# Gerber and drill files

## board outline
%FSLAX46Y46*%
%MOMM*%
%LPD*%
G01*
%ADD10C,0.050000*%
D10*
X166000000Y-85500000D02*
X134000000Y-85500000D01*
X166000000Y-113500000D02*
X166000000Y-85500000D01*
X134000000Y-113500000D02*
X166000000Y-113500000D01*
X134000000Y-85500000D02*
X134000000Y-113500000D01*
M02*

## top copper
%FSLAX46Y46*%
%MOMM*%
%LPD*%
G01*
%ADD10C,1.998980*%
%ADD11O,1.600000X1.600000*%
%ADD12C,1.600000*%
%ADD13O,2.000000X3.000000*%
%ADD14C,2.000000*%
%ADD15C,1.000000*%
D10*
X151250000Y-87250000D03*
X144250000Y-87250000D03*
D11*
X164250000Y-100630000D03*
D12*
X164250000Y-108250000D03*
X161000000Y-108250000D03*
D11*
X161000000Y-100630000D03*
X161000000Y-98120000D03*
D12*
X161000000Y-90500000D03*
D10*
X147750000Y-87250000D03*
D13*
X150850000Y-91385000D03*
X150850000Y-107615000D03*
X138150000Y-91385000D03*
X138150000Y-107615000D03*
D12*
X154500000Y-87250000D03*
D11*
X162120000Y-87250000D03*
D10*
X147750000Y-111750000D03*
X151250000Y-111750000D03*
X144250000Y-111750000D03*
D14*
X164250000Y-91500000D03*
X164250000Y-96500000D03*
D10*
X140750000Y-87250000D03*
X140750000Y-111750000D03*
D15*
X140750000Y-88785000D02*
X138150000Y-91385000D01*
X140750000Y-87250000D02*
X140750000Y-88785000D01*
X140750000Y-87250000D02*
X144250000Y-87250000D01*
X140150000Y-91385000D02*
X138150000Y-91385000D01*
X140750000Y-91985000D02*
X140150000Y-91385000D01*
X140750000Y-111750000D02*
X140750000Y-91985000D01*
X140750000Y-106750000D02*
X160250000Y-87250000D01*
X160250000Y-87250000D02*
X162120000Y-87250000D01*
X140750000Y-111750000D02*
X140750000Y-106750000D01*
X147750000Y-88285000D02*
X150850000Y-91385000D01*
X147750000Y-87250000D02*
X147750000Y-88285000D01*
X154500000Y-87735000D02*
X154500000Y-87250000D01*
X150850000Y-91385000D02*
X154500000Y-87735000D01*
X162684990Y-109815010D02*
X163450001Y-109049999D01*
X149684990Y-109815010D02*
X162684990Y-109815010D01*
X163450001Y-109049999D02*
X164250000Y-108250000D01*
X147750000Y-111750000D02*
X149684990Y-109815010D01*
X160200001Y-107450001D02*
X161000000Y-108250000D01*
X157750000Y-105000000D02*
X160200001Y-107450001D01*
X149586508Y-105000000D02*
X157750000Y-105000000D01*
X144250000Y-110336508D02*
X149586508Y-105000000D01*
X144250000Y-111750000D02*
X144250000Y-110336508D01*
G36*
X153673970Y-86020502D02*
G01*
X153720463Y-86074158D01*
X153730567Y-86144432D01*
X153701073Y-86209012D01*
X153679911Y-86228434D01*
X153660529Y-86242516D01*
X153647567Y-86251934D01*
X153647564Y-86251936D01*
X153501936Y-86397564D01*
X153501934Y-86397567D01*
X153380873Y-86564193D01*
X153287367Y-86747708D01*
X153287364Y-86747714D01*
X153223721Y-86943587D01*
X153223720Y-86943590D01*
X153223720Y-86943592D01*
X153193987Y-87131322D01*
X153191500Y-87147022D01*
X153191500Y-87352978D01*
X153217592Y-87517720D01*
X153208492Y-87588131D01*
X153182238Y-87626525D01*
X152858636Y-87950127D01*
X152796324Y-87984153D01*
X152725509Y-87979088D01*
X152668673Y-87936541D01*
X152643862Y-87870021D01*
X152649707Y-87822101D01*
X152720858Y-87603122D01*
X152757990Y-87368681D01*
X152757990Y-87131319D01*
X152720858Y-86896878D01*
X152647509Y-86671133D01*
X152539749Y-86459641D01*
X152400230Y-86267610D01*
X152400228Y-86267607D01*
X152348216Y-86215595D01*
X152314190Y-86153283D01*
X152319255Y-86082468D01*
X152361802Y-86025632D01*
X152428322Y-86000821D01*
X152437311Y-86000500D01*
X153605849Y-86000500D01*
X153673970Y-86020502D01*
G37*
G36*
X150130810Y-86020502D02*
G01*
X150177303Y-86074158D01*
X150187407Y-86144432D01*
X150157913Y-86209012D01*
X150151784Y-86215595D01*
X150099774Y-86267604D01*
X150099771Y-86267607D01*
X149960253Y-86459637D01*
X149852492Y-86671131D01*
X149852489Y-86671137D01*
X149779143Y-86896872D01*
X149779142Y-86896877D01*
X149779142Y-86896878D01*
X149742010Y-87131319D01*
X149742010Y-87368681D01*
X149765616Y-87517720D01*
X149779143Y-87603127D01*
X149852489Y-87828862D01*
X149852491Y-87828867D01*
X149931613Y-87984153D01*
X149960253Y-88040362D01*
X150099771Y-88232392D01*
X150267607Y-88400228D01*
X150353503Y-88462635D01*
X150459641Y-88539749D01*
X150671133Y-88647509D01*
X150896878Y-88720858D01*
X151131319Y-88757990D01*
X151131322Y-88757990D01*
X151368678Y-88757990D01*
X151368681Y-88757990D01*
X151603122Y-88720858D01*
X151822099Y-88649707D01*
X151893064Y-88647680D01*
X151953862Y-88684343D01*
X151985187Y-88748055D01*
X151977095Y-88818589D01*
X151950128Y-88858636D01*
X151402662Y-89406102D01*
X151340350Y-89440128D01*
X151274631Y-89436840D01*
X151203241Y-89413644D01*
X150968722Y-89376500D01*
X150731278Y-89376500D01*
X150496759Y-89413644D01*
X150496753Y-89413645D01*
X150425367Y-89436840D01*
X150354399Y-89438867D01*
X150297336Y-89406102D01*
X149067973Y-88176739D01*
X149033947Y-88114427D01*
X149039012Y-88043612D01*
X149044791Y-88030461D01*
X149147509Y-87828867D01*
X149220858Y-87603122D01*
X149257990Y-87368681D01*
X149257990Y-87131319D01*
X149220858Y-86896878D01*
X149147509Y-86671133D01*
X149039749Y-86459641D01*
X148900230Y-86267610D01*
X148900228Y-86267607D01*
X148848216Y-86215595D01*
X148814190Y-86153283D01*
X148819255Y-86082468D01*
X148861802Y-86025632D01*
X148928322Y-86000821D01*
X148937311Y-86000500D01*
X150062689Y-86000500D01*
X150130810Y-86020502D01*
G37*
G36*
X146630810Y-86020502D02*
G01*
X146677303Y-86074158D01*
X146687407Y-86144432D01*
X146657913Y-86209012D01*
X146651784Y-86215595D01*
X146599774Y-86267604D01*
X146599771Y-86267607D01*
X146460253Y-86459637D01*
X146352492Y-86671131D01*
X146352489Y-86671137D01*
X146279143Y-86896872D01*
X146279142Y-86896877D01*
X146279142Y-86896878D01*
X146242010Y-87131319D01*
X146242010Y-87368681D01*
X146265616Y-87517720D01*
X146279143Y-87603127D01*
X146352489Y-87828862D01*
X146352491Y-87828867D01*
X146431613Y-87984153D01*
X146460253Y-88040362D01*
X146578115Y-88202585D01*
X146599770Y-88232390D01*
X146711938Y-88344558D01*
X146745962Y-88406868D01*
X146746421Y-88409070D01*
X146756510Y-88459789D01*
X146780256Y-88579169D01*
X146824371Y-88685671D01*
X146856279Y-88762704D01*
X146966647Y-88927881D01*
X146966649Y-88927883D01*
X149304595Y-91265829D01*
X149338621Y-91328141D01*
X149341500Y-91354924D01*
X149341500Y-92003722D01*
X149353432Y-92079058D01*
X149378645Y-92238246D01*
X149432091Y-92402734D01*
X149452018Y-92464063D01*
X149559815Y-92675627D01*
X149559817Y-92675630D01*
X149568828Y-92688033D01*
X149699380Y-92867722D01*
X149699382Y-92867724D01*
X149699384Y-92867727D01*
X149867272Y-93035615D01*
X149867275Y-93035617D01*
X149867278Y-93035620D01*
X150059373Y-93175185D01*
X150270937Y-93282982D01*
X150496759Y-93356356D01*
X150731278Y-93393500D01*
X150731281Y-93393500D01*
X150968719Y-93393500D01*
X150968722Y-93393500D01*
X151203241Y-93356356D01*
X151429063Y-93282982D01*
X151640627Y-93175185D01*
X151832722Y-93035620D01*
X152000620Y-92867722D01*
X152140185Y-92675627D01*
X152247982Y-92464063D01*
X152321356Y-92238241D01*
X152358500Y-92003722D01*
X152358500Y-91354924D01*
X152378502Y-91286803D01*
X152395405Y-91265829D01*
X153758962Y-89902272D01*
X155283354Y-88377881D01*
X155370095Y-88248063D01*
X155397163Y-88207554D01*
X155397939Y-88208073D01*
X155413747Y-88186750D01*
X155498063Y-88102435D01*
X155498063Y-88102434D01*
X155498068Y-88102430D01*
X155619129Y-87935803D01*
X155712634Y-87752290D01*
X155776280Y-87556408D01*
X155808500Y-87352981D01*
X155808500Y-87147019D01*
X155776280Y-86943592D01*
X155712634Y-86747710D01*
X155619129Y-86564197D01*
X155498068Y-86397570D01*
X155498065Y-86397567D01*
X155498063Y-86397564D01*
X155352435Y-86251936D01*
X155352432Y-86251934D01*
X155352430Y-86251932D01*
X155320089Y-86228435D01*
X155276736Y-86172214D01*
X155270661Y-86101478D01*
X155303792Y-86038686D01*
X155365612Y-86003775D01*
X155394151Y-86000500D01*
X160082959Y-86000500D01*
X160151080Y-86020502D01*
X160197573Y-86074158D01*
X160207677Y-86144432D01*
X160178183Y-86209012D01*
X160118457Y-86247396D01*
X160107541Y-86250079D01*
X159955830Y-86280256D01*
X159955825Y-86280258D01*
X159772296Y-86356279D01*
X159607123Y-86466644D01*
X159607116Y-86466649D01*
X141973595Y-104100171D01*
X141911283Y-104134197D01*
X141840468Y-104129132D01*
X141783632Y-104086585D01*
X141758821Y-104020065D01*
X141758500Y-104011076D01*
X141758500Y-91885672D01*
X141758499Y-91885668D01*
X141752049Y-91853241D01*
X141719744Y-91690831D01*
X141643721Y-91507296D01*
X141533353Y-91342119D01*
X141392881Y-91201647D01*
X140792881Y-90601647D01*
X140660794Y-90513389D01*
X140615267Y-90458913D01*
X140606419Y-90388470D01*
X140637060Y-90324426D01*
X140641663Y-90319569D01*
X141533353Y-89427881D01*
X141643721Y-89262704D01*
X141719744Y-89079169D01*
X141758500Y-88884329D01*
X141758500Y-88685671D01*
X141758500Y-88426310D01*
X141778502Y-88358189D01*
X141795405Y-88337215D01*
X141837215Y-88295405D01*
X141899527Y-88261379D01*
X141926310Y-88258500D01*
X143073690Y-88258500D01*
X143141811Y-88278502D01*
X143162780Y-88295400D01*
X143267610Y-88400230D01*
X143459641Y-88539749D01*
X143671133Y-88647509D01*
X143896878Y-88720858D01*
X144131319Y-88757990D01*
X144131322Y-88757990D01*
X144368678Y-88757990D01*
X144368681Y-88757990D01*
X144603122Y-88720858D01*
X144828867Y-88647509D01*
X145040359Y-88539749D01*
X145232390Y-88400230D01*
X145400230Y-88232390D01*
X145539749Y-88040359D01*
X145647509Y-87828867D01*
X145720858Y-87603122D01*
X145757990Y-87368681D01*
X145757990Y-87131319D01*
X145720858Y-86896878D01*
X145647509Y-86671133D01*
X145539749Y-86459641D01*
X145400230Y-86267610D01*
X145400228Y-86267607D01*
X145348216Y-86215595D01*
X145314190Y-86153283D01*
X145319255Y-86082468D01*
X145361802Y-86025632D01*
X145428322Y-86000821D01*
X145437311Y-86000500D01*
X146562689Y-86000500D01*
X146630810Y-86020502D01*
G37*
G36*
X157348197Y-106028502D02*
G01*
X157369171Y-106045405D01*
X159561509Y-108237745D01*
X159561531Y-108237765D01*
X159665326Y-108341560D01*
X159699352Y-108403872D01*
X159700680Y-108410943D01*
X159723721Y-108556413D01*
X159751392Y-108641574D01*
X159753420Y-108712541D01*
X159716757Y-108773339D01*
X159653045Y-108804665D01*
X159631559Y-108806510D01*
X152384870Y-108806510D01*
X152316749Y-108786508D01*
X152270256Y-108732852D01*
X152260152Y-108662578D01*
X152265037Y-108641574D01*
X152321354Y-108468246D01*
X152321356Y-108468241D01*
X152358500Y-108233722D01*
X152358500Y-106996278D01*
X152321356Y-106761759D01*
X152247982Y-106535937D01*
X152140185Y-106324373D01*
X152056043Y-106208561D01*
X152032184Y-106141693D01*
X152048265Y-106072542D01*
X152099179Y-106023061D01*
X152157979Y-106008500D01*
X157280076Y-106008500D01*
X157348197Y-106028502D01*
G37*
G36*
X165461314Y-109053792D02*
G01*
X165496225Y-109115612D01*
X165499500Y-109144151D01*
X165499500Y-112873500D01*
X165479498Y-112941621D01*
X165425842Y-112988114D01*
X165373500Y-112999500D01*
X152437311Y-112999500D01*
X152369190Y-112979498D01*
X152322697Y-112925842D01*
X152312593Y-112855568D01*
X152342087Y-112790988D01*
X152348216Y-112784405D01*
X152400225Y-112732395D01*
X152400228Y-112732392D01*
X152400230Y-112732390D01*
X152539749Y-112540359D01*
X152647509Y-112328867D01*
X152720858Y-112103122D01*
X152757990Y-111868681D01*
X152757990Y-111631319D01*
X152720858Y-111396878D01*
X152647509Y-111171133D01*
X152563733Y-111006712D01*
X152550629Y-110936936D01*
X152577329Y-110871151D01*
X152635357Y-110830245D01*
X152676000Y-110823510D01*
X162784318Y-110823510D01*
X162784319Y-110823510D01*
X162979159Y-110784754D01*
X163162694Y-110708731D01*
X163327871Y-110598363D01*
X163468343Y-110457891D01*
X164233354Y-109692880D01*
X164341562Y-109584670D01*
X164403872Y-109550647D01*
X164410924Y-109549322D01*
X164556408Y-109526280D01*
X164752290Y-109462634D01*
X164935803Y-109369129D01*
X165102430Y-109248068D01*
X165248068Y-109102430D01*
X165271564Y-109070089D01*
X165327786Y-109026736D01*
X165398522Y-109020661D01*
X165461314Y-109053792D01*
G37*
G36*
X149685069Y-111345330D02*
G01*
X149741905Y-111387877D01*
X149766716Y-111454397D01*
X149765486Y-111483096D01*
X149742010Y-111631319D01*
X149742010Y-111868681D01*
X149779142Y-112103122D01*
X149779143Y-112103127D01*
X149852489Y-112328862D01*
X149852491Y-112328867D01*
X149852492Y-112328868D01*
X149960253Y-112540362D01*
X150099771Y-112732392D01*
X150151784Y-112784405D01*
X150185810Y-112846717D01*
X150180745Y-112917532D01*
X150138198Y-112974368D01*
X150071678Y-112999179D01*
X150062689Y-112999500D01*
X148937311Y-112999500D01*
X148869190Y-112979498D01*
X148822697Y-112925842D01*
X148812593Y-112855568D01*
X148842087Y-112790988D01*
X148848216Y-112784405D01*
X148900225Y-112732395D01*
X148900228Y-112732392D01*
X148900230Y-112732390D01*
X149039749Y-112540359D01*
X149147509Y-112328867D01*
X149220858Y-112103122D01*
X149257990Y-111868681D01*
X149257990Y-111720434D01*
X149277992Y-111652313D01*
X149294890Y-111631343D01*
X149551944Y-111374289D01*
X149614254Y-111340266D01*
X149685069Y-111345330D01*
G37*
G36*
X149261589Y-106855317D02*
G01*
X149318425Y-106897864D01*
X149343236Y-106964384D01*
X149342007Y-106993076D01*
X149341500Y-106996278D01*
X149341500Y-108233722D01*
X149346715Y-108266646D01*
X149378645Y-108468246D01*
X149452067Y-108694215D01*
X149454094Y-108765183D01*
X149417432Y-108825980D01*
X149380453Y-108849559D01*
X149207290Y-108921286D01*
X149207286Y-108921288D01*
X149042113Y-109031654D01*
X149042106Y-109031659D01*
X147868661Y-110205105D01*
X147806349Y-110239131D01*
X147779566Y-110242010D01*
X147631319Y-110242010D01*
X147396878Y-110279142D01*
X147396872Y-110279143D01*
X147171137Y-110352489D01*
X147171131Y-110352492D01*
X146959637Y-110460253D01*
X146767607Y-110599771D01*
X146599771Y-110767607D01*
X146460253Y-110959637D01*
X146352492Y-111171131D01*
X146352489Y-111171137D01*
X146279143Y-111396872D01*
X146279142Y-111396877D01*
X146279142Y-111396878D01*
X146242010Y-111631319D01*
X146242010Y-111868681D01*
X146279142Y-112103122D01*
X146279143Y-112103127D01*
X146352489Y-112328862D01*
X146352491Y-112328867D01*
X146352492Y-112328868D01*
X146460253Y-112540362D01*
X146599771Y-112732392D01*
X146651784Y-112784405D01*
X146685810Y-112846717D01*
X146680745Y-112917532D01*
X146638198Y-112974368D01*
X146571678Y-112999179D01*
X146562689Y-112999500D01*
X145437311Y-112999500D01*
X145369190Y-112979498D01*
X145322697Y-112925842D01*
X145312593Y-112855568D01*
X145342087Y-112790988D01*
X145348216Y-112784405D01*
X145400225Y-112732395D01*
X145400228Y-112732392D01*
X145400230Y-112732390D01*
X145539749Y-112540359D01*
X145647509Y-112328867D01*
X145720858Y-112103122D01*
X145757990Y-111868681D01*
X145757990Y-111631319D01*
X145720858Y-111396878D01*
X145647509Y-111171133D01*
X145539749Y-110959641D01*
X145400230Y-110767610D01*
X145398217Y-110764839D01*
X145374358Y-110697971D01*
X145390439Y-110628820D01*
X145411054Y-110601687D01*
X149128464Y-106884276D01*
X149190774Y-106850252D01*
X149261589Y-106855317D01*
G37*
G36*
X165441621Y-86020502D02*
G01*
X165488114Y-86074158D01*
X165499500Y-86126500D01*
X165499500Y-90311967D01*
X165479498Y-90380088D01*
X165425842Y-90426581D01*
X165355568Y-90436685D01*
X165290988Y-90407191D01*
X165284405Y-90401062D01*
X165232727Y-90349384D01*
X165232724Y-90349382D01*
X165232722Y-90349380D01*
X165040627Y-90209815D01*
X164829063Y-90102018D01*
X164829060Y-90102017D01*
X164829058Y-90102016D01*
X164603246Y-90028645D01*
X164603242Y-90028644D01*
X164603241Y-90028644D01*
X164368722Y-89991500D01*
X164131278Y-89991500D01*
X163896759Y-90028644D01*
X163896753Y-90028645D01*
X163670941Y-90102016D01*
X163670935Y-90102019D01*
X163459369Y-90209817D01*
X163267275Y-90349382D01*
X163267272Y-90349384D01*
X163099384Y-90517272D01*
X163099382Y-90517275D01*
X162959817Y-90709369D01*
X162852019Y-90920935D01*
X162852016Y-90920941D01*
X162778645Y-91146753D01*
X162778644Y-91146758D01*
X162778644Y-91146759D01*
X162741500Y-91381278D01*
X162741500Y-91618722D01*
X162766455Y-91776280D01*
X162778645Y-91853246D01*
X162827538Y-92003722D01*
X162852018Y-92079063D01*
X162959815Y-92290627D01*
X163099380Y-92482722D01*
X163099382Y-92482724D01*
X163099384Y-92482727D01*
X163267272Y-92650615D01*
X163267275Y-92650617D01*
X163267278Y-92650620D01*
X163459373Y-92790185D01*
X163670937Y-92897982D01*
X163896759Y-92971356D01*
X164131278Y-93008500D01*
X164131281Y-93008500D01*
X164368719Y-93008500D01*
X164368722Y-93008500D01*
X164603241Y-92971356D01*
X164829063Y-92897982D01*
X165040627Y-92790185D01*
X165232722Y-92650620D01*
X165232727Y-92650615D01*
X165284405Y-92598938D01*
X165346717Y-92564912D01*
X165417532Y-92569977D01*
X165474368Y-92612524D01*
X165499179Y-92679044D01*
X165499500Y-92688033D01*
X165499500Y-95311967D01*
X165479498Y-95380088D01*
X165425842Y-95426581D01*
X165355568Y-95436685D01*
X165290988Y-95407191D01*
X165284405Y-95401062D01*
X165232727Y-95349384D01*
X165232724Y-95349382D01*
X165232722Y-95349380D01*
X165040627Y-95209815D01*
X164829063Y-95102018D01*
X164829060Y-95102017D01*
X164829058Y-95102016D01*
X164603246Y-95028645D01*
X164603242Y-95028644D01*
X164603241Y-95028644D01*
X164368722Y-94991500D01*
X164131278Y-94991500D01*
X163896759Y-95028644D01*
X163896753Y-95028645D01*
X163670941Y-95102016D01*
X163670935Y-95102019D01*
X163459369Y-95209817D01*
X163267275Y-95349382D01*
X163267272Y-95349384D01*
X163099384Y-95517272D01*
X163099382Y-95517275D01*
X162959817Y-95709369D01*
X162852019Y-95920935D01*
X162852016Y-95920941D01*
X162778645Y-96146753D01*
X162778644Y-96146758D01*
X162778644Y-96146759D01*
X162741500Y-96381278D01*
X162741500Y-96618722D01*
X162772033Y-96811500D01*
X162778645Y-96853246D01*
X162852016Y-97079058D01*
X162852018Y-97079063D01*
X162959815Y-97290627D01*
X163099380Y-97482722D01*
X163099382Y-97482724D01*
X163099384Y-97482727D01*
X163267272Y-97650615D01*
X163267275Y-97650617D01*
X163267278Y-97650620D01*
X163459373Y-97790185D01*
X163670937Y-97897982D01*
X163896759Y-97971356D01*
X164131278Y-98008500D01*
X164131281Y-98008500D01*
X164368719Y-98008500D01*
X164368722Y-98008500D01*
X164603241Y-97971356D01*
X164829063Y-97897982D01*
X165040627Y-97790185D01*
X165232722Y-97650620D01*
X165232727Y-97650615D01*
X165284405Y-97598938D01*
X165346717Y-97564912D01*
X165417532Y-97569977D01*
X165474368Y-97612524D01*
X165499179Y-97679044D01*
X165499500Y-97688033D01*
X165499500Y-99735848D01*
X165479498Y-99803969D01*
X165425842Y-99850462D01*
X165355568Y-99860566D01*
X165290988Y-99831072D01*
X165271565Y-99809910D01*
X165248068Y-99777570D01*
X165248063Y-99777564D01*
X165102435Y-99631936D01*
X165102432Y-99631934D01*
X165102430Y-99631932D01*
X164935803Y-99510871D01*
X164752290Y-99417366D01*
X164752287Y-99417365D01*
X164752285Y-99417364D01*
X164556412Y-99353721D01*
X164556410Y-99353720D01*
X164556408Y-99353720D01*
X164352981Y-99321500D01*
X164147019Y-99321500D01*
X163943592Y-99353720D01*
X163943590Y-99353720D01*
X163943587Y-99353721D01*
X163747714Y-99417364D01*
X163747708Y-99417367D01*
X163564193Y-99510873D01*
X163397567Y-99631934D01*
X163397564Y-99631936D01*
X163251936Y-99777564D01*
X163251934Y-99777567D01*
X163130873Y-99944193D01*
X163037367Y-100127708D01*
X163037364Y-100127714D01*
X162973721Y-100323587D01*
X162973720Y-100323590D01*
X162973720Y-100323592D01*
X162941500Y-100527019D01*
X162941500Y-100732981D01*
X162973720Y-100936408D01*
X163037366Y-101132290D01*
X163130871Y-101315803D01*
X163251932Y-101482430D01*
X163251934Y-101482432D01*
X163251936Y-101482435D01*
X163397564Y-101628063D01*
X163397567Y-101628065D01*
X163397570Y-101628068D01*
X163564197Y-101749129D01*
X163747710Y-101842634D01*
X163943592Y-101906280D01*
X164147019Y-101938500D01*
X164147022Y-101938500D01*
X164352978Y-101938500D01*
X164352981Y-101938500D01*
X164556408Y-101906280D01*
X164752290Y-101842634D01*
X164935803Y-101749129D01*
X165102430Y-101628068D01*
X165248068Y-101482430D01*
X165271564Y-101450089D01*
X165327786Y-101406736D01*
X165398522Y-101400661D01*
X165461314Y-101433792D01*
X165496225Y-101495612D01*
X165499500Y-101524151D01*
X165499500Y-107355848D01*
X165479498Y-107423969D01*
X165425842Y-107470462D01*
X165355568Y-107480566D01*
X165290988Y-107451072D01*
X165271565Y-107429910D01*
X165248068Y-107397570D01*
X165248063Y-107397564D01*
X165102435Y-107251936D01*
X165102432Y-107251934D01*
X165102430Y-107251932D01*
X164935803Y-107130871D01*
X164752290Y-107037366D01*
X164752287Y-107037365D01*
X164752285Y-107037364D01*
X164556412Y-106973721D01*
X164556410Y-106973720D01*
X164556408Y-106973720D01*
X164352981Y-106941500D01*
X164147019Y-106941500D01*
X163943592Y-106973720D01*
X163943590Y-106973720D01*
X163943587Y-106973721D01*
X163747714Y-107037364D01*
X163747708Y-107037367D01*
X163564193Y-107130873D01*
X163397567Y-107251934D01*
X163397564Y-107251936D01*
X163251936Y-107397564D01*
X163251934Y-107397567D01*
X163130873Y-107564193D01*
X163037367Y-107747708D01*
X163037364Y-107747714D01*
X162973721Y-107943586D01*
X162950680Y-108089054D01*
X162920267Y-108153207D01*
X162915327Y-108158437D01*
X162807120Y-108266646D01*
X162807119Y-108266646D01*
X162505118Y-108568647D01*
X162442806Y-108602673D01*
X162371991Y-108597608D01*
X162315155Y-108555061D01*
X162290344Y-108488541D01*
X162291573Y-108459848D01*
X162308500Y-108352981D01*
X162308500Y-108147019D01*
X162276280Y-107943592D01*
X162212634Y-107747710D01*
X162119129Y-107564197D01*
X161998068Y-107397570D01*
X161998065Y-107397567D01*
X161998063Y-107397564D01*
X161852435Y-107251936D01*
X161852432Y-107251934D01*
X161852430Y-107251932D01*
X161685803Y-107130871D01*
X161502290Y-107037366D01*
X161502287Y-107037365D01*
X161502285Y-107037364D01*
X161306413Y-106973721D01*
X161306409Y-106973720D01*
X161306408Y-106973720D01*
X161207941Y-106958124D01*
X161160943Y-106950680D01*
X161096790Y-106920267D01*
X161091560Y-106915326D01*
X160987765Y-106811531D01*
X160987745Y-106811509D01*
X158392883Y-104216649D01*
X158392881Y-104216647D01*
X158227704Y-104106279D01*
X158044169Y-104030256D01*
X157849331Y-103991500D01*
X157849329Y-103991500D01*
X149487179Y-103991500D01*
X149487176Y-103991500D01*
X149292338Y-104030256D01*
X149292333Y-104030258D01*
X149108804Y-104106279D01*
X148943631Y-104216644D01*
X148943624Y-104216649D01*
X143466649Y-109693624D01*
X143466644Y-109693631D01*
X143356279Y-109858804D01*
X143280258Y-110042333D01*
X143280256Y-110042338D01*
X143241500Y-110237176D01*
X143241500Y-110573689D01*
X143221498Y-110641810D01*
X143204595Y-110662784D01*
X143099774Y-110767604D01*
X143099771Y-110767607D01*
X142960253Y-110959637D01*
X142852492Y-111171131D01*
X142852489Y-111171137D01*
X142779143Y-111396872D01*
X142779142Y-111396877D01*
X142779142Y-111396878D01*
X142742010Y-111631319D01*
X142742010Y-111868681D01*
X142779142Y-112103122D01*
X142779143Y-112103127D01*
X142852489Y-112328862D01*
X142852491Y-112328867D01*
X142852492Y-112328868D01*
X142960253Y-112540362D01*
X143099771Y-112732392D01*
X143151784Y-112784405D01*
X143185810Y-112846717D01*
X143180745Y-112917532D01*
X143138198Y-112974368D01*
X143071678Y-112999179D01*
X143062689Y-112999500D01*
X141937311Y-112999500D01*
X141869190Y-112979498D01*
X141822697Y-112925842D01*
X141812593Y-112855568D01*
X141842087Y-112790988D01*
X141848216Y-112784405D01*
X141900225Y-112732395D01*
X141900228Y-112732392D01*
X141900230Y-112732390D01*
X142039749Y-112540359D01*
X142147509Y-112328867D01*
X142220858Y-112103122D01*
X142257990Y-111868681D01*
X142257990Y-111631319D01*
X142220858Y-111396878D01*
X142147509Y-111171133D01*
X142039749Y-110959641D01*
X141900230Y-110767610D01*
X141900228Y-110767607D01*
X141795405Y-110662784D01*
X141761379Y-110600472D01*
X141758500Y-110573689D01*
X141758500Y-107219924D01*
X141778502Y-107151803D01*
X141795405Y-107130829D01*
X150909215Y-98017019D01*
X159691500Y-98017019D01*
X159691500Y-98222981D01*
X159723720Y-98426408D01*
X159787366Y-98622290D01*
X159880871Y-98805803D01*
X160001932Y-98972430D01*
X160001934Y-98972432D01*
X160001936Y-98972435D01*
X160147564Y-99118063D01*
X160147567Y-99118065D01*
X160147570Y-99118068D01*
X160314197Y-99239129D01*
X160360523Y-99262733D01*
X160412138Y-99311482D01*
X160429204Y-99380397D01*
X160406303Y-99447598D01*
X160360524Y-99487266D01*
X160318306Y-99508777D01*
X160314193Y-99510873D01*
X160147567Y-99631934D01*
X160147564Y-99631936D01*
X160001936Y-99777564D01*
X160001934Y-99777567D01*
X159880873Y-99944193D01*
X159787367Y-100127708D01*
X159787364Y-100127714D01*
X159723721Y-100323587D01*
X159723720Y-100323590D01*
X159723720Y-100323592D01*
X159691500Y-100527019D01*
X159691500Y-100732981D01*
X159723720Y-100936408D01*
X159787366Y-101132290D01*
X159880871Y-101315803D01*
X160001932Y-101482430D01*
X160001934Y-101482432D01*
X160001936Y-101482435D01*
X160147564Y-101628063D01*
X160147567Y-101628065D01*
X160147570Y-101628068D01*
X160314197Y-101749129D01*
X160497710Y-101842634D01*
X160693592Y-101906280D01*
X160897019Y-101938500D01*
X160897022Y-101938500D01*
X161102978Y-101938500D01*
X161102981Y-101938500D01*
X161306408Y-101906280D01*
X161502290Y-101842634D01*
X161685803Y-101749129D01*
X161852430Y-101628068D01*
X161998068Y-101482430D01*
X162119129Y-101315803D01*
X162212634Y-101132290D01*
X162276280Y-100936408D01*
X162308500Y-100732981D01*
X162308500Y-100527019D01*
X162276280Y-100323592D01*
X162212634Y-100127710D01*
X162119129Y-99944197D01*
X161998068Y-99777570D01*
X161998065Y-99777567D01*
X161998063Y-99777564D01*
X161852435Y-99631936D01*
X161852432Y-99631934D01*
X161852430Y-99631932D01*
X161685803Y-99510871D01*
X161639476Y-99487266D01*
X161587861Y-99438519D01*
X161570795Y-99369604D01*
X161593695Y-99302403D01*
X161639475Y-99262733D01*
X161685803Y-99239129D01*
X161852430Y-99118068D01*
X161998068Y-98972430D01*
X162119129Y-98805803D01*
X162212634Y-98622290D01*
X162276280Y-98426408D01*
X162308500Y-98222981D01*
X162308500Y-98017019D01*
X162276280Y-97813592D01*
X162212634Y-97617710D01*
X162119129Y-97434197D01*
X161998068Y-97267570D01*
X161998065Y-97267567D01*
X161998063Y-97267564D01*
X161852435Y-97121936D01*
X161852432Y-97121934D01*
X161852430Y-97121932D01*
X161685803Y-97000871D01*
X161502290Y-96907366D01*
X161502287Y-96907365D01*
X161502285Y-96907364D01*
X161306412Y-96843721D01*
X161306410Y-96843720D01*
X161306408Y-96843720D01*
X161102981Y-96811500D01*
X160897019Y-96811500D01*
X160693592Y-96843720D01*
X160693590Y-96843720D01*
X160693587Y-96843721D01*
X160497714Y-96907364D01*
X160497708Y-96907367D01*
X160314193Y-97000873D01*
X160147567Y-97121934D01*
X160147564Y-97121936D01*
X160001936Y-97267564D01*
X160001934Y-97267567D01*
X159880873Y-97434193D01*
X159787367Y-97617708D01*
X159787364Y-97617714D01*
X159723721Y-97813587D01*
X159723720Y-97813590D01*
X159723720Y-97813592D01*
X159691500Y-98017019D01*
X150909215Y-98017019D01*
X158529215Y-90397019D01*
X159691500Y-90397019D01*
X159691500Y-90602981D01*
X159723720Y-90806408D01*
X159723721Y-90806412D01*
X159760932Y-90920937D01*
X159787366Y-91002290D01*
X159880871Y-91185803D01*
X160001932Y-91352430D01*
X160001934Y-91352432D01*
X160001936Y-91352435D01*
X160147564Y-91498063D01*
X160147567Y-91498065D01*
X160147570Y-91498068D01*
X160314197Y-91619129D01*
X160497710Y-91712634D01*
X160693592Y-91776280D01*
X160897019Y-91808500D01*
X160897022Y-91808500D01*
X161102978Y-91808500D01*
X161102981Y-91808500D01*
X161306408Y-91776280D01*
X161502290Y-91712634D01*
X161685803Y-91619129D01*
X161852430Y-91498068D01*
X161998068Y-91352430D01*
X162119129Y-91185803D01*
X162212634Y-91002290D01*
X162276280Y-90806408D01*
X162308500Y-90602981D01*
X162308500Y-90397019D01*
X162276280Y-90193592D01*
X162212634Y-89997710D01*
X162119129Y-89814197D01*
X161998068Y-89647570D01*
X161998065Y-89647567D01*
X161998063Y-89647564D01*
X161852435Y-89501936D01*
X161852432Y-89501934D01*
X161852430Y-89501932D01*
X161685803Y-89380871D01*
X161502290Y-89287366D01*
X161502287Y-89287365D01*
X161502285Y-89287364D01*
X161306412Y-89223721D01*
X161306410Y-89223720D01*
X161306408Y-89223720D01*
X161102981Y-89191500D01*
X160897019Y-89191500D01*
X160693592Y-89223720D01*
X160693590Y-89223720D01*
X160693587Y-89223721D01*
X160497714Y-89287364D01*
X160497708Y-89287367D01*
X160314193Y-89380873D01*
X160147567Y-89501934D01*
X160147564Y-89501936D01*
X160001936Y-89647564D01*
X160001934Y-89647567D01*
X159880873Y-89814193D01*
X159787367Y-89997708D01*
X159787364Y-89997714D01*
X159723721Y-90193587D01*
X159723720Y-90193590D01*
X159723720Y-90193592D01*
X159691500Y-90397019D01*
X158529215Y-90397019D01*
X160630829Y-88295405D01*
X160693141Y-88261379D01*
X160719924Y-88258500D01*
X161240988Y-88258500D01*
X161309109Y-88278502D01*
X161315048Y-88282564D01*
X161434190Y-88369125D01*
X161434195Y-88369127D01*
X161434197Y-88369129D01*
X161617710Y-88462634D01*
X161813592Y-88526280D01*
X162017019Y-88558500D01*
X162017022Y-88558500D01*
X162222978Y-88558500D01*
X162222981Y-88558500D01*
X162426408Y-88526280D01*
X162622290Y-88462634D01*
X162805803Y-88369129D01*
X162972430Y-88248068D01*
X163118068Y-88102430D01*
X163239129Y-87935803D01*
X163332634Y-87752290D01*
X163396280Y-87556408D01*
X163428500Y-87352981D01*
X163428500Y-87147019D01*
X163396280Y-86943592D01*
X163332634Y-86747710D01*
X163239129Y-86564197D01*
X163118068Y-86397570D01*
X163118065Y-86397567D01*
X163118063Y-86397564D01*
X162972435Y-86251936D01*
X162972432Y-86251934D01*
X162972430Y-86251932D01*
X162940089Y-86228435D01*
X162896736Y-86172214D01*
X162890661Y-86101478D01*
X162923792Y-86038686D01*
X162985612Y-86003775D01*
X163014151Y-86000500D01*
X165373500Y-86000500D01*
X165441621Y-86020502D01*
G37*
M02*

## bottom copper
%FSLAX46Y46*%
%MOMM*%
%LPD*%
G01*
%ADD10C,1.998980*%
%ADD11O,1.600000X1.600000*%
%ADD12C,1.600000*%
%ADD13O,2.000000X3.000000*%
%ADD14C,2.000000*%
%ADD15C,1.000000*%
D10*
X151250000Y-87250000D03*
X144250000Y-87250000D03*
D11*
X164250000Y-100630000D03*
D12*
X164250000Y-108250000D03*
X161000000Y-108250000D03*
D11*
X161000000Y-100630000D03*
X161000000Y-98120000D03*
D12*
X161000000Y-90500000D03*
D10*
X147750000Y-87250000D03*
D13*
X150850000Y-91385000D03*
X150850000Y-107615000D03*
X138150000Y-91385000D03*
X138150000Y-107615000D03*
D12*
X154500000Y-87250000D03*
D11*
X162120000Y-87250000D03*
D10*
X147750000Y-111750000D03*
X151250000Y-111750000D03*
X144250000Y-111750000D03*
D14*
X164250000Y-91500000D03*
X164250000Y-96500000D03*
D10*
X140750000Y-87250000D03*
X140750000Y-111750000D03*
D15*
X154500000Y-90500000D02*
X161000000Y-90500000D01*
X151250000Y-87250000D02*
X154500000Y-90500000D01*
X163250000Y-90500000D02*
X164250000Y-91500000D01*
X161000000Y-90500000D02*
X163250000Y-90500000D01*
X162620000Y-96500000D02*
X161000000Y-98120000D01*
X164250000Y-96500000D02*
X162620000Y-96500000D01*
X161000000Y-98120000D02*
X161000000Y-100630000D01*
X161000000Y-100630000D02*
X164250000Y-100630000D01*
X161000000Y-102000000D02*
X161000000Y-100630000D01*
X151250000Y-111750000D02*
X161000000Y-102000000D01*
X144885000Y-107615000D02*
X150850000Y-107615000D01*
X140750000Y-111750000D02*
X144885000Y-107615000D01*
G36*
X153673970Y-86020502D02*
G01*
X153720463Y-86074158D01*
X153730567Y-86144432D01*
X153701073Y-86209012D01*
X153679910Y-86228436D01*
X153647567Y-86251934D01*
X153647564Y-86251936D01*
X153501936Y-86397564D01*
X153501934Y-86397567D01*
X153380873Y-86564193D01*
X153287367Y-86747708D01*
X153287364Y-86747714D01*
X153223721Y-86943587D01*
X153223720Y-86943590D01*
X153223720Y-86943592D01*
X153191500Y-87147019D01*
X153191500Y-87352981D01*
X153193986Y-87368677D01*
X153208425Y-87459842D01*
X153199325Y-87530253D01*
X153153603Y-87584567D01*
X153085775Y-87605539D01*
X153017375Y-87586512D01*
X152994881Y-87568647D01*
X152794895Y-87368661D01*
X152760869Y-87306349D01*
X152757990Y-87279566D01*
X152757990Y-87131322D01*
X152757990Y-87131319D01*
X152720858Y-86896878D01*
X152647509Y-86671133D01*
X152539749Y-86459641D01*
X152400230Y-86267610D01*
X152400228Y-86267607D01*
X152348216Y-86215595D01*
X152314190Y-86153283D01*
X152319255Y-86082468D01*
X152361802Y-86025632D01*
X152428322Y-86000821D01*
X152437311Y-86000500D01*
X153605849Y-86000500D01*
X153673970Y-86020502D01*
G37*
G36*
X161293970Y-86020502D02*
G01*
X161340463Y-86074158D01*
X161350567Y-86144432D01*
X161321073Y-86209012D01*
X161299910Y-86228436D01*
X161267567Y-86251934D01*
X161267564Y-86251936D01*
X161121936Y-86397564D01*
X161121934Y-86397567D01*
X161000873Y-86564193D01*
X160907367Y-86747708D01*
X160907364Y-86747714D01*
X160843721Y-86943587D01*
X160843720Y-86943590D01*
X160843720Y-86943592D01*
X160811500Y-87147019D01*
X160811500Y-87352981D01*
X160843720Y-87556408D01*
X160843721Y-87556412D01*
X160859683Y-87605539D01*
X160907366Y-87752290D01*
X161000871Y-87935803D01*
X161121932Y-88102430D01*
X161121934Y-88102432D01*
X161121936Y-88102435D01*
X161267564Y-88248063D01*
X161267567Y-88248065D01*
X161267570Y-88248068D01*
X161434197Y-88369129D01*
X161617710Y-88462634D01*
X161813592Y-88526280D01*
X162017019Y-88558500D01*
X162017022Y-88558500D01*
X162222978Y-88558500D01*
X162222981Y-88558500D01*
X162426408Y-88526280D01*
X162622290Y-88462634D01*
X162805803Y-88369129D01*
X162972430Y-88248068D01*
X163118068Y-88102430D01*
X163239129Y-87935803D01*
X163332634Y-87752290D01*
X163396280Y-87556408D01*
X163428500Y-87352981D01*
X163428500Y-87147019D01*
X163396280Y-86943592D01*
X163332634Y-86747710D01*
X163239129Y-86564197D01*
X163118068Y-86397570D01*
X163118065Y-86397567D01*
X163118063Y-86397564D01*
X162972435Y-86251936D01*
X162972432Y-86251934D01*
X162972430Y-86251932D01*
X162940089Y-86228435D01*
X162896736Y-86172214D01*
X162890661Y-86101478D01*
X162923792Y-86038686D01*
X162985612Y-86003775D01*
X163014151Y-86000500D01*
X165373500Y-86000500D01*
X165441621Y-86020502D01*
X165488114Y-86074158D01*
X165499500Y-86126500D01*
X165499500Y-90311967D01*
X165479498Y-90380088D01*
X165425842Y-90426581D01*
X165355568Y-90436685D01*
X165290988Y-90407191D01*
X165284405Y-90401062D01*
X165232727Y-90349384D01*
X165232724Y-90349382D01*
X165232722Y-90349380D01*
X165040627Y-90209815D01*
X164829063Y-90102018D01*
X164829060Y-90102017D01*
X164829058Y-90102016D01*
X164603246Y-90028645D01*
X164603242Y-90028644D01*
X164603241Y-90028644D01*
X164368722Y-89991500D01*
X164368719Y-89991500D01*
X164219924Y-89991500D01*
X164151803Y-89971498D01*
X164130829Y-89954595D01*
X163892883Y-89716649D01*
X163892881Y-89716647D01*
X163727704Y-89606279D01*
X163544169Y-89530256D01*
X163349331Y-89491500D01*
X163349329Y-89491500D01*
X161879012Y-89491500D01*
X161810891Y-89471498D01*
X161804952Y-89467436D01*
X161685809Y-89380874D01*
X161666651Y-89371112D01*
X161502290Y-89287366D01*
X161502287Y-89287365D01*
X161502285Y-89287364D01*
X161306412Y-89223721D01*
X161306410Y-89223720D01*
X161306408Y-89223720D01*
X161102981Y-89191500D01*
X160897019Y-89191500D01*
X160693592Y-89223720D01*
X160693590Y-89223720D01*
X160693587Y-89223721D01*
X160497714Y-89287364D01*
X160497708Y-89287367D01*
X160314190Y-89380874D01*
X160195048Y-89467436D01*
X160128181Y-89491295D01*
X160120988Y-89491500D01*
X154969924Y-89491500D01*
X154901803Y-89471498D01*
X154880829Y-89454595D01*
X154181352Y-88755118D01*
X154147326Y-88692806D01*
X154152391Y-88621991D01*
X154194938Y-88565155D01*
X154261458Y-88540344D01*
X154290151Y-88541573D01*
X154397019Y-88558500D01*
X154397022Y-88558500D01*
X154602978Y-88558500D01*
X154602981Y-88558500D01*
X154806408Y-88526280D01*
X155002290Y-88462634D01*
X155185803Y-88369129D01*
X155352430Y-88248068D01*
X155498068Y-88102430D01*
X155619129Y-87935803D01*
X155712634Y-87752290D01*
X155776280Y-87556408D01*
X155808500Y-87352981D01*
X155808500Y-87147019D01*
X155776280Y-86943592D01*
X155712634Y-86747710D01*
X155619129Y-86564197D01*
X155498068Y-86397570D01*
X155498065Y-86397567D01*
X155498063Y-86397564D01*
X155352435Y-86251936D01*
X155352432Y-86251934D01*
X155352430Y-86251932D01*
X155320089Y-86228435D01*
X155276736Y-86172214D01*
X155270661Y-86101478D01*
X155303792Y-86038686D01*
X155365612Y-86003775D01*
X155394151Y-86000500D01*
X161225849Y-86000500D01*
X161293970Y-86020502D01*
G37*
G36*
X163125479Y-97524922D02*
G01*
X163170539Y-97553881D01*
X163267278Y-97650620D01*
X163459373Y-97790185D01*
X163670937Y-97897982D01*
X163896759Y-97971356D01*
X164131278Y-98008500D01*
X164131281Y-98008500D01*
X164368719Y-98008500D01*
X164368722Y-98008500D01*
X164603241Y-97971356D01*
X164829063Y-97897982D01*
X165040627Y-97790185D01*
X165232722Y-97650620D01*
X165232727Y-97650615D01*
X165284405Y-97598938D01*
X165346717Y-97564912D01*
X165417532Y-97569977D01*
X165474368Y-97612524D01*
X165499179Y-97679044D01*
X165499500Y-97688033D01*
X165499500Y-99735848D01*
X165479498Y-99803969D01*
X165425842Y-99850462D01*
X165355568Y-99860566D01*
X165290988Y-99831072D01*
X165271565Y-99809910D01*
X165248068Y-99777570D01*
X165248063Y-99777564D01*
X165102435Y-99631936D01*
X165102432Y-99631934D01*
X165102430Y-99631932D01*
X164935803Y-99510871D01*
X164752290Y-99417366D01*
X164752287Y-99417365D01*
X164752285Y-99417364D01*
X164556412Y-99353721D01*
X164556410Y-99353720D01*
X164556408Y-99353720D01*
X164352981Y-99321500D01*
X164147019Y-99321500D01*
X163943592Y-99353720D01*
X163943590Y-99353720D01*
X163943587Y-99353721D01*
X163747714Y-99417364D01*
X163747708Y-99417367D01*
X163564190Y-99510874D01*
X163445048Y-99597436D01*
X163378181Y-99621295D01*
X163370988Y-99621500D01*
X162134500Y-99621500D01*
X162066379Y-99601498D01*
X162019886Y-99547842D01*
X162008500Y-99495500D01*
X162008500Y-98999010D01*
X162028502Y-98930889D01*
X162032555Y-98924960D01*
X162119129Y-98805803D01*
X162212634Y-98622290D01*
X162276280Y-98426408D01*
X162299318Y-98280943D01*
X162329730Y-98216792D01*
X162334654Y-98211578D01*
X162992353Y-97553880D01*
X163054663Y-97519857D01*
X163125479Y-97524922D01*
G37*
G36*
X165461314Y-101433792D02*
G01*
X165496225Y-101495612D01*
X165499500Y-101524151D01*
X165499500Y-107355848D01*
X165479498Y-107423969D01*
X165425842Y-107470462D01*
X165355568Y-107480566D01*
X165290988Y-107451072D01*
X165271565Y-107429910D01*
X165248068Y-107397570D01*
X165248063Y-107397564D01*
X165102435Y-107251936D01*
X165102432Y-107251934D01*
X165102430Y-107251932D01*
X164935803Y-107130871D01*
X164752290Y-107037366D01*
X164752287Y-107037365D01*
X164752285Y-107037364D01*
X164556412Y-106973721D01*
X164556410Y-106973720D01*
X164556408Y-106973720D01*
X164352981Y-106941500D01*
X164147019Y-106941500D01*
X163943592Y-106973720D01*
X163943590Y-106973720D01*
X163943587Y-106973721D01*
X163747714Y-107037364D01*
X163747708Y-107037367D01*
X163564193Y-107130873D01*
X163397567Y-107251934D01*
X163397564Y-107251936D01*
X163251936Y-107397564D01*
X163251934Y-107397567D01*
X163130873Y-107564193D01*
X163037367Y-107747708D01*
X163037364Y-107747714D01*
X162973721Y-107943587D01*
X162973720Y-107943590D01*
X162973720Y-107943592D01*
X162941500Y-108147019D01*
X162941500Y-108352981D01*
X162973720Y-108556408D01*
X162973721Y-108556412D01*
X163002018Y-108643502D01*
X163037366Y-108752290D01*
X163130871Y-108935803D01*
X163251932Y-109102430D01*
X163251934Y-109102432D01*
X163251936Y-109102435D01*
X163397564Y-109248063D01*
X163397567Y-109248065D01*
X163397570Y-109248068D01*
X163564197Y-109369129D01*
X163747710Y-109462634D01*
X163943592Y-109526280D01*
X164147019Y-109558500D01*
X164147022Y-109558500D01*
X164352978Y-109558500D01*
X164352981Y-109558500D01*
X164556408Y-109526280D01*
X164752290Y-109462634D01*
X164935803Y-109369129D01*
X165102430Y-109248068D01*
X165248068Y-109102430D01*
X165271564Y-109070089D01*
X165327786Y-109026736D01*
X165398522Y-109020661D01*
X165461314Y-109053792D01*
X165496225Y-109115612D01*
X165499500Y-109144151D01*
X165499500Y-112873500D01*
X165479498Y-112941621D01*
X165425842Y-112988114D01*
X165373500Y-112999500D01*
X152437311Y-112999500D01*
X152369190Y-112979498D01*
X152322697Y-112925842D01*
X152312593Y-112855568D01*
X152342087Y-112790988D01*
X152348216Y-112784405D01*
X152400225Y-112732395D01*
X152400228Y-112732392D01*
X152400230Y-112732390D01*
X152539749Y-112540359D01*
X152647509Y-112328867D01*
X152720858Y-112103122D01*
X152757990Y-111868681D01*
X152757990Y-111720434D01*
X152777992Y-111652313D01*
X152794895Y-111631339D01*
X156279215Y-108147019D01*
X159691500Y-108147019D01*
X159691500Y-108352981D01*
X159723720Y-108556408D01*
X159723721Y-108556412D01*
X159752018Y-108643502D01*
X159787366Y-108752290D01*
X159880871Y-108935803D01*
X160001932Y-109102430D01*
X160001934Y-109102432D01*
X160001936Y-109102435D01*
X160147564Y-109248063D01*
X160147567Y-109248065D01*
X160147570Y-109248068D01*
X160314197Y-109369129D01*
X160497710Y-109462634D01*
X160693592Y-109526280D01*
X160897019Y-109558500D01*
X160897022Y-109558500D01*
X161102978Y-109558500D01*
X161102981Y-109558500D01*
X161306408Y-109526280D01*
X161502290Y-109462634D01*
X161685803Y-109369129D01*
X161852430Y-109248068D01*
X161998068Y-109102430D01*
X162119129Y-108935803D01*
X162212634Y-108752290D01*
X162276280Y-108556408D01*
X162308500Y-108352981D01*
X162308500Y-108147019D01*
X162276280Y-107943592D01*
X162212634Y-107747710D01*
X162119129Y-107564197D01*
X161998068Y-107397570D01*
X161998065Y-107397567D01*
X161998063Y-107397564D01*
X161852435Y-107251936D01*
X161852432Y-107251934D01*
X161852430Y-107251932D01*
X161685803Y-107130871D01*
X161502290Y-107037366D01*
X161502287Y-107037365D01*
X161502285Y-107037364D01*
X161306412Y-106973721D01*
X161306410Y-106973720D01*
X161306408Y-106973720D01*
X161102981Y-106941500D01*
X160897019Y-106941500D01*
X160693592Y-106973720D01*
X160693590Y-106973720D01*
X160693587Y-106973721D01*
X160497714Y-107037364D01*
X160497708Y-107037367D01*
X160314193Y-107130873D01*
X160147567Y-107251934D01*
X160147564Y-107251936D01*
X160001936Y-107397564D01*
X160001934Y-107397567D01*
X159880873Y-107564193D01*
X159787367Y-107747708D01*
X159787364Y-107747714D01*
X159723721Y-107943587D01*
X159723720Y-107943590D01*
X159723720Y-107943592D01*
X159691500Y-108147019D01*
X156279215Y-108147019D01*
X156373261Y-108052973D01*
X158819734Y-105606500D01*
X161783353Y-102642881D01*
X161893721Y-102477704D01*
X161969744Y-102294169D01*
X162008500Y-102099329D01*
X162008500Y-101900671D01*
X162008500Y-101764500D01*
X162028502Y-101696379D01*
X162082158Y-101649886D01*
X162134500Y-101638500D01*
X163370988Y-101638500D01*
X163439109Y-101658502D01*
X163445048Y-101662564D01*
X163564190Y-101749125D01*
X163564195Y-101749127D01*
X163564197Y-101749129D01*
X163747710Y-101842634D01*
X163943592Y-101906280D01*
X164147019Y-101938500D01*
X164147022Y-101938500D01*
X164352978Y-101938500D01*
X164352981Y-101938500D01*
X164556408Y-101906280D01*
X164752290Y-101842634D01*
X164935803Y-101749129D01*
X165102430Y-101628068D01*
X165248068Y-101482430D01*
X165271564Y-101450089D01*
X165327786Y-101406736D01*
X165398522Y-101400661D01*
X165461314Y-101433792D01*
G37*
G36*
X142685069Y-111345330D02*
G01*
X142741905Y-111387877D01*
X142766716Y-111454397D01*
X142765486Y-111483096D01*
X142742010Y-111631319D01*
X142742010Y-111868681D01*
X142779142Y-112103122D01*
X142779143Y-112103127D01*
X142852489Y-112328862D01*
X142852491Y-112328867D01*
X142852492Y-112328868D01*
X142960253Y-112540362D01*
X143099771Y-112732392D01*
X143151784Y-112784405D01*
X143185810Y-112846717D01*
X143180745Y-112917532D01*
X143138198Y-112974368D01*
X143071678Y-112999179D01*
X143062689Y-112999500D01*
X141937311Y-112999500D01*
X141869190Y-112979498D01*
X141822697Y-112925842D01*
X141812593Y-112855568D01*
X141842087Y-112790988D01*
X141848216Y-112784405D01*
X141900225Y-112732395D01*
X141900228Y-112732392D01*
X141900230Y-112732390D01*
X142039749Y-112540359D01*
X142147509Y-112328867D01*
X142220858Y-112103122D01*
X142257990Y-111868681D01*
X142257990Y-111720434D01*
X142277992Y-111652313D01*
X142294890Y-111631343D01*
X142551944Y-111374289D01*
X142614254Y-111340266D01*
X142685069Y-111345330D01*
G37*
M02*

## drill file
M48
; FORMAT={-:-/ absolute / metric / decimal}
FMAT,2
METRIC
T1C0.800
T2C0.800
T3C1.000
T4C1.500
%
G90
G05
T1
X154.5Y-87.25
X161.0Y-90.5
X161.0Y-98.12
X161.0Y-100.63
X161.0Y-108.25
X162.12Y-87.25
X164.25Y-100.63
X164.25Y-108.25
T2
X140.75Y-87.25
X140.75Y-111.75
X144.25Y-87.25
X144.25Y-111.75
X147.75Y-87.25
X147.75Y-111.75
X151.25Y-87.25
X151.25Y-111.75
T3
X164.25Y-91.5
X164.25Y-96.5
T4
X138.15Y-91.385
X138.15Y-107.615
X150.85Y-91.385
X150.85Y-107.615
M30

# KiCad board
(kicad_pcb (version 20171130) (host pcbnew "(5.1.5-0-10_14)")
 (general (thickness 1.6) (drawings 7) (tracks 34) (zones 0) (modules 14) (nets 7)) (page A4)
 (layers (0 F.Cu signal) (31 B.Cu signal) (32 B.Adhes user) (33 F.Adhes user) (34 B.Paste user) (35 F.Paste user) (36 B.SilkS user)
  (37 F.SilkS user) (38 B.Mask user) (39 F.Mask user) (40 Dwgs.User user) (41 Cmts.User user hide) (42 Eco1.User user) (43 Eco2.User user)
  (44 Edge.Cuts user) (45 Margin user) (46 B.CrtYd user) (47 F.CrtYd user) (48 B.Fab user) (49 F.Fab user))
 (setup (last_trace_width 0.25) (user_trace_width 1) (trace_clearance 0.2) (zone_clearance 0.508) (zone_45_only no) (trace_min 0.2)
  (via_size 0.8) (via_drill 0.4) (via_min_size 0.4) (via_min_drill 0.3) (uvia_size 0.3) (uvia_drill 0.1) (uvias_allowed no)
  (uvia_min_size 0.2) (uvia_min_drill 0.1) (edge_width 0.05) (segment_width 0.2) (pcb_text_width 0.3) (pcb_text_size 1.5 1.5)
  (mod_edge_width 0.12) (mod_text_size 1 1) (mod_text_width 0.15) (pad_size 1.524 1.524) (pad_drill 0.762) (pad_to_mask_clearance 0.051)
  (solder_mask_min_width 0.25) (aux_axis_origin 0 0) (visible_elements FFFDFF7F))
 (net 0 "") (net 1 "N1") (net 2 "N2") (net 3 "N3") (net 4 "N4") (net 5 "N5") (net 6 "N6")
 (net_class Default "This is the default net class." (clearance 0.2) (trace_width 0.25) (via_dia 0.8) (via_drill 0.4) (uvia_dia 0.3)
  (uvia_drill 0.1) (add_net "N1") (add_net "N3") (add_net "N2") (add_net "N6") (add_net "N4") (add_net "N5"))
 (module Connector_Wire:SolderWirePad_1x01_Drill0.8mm (layer F.Cu) (at 151.25 87.25 180)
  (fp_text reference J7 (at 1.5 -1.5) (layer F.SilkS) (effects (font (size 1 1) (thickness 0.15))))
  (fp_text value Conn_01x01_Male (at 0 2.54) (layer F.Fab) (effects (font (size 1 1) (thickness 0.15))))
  (pad 1 thru_hole circle (at 0 0 180) (size 1.99898 1.99898) (drill 0.8001) (layers *.Cu *.Mask) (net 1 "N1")))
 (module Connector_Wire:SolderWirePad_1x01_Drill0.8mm (layer F.Cu) (at 144.25 87.25)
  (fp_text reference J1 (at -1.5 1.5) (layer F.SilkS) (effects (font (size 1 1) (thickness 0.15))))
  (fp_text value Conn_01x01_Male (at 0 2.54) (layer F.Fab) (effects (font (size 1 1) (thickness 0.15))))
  (pad 1 thru_hole circle (at 0 0) (size 1.99898 1.99898) (drill 0.8001) (layers *.Cu *.Mask) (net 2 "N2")))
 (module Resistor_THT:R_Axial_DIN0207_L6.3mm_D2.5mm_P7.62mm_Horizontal (layer F.Cu) (at 164.25 108.25 90)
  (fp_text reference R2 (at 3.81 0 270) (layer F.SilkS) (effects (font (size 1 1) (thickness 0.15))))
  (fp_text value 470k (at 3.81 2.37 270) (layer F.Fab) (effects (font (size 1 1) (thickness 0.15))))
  (pad 2 thru_hole oval (at 7.62 0 90) (size 1.6 1.6) (drill 0.8) (layers *.Cu *.Mask) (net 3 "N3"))
  (pad 1 thru_hole circle (at 0 0 90) (size 1.6 1.6) (drill 0.8) (layers *.Cu *.Mask) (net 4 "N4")))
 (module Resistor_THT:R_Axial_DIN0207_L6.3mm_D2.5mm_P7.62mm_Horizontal (layer F.Cu) (at 161 108.25 90)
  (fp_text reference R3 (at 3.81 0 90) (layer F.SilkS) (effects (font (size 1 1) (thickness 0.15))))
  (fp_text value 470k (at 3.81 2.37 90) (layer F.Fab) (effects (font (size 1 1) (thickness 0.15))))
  (pad 1 thru_hole circle (at 0 0 90) (size 1.6 1.6) (drill 0.8) (layers *.Cu *.Mask) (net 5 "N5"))
  (pad 2 thru_hole oval (at 7.62 0 90) (size 1.6 1.6) (drill 0.8) (layers *.Cu *.Mask) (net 3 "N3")))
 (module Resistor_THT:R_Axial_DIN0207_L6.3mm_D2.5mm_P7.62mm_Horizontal (layer F.Cu) (at 161 90.5 270)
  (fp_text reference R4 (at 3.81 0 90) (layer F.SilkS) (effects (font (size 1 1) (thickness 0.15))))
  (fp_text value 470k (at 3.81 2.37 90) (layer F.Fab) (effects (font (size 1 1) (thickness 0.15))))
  (pad 2 thru_hole oval (at 7.62 0 270) (size 1.6 1.6) (drill 0.8) (layers *.Cu *.Mask) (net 3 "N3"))
  (pad 1 thru_hole circle (at 0 0 270) (size 1.6 1.6) (drill 0.8) (layers *.Cu *.Mask) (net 1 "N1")))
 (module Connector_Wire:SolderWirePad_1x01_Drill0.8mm (layer F.Cu) (at 147.75 87.25)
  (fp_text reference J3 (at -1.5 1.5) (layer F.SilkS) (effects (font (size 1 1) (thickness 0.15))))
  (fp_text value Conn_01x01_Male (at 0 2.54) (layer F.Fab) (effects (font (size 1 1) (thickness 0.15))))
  (pad 1 thru_hole circle (at 0 0) (size 1.99898 1.99898) (drill 0.8001) (layers *.Cu *.Mask) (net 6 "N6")))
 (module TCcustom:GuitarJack (layer B.Cu) (at 144.5 99.5 180)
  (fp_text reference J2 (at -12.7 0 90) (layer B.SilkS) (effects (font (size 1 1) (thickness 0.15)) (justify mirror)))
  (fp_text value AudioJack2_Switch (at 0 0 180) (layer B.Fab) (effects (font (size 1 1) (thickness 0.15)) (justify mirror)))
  (pad T thru_hole oval (at -6.35 8.115 180) (size 2 3) (drill 1.5) (layers *.Cu *.Mask) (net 6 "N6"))
  (pad TN thru_hole oval (at -6.35 -8.115 180) (size 2 3) (drill 1.5) (layers *.Cu *.Mask) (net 2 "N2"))
  (pad S thru_hole oval (at 6.35 8.115 180) (size 2 3) (drill 1.5) (layers *.Cu *.Mask) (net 2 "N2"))
  (pad SN thru_hole oval (at 6.35 -8.115 180) (size 2 3) (drill 1.5) (layers *.Cu *.Mask)))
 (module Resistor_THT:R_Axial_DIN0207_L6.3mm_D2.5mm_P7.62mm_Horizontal (layer F.Cu) (at 154.5 87.25)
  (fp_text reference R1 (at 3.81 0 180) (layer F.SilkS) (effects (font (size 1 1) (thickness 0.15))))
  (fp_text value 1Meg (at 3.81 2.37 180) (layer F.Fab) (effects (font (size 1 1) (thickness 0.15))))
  (pad 1 thru_hole circle (at 0 0) (size 1.6 1.6) (drill 0.8) (layers *.Cu *.Mask) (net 6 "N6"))
  (pad 2 thru_hole oval (at 7.62 0) (size 1.6 1.6) (drill 0.8) (layers *.Cu *.Mask) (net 2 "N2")))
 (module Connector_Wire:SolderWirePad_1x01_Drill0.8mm (layer F.Cu) (at 147.75 111.75)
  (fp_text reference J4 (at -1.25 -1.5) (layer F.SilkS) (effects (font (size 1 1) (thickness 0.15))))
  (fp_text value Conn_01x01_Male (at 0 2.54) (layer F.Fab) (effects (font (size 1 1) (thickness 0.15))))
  (pad 1 thru_hole circle (at 0 0) (size 1.99898 1.99898) (drill 0.8001) (layers *.Cu *.Mask) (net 4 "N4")))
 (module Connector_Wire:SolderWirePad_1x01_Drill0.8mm (layer F.Cu) (at 151.25 111.75 180)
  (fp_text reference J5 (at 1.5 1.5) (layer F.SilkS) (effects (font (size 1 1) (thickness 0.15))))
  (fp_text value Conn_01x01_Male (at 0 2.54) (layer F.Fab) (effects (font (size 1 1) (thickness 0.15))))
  (pad 1 thru_hole circle (at 0 0 180) (size 1.99898 1.99898) (drill 0.8001) (layers *.Cu *.Mask) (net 3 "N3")))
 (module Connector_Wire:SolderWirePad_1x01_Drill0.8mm (layer F.Cu) (at 144.25 111.75 180)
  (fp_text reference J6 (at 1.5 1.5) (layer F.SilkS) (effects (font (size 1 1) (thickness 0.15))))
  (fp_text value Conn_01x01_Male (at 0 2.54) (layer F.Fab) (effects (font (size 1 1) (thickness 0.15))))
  (pad 1 thru_hole circle (at 0 0 180) (size 1.99898 1.99898) (drill 0.8001) (layers *.Cu *.Mask) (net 5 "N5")))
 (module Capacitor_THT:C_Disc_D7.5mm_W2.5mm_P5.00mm (layer F.Cu) (at 164.25 91.5 270)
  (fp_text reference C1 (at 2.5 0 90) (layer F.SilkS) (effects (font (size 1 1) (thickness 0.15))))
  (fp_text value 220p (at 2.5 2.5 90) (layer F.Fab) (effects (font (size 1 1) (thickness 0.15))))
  (pad 1 thru_hole circle (at 0 0 270) (size 2 2) (drill 1) (layers *.Cu *.Mask) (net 1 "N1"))
  (pad 2 thru_hole circle (at 5 0 270) (size 2 2) (drill 1) (layers *.Cu *.Mask) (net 3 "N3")))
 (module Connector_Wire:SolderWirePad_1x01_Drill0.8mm (layer F.Cu) (at 140.75 87.25)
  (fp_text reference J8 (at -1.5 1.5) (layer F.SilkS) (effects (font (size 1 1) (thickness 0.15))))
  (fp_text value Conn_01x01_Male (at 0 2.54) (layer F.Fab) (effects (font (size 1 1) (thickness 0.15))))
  (pad 1 thru_hole circle (at 0 0) (size 1.99898 1.99898) (drill 0.8001) (layers *.Cu *.Mask) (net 2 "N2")))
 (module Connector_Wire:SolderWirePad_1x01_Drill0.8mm (layer F.Cu) (at 140.75 111.75)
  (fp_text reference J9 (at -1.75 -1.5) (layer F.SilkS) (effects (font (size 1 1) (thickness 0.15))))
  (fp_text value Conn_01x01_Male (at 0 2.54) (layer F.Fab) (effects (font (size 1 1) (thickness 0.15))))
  (pad 1 thru_hole circle (at 0 0) (size 1.99898 1.99898) (drill 0.8001) (layers *.Cu *.Mask) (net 2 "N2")))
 (gr_line (start 166 85.5) (end 134 85.5) (layer Edge.Cuts) (width 0.05))
 (gr_line (start 166 113.5) (end 166 85.5) (layer Edge.Cuts) (width 0.05))
 (gr_line (start 134 113.5) (end 166 113.5) (layer Edge.Cuts) (width 0.05))
 (gr_line (start 134 85.5) (end 134 113.5) (layer Edge.Cuts) (width 0.05))
 (segment (start 154.5 90.5) (end 161 90.5) (width 1) (layer B.Cu) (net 1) (status 20))
 (segment (start 151.25 87.25) (end 154.5 90.5) (width 1) (layer B.Cu) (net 1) (status 10))
 (segment (start 163.25 90.5) (end 164.25 91.5) (width 1) (layer B.Cu) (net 1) (status 20))
 (segment (start 161 90.5) (end 163.25 90.5) (width 1) (layer B.Cu) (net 1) (status 10))
 (segment (start 162.62 96.5) (end 161 98.12) (width 1) (layer B.Cu) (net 3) (status 20))
 (segment (start 164.25 96.5) (end 162.62 96.5) (width 1) (layer B.Cu) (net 3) (status 10))
 (segment (start 161 98.12) (end 161 100.63) (width 1) (layer B.Cu) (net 3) (status 30))
 (segment (start 161 100.63) (end 164.25 100.63) (width 1) (layer B.Cu) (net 3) (status 30))
 (segment (start 161 102) (end 161 100.63) (width 1) (layer B.Cu) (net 3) (status 20))
 (segment (start 151.25 111.75) (end 161 102) (width 1) (layer B.Cu) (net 3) (status 10))
 (segment (start 140.75 88.785) (end 138.15 91.385) (width 1) (layer F.Cu) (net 2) (status 20))
 (segment (start 140.75 87.25) (end 140.75 88.785) (width 1) (layer F.Cu) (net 2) (status 10))
 (segment (start 140.75 87.25) (end 144.25 87.25) (width 1) (layer F.Cu) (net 2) (status 30))
 (segment (start 140.15 91.385) (end 138.15 91.385) (width 1) (layer F.Cu) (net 2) (status 20))
 (segment (start 140.75 91.985) (end 140.15 91.385) (width 1) (layer F.Cu) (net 2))
 (segment (start 140.75 111.75) (end 140.75 91.985) (width 1) (layer F.Cu) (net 2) (status 10))
 (segment (start 140.75 106.75) (end 160.25 87.25) (width 1) (layer F.Cu) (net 2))
 (segment (start 160.25 87.25) (end 162.12 87.25) (width 1) (layer F.Cu) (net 2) (status 20))
 (segment (start 140.75 111.75) (end 140.75 106.75) (width 1) (layer F.Cu) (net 2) (status 10))
 (segment (start 144.885 107.615) (end 150.85 107.615) (width 1) (layer B.Cu) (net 2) (status 20))
 (segment (start 140.75 111.75) (end 144.885 107.615) (width 1) (layer B.Cu) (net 2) (status 10))
 (segment (start 147.75 88.285) (end 150.85 91.385) (width 1) (layer F.Cu) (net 6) (status 20))
 (segment (start 147.75 87.25) (end 147.75 88.285) (width 1) (layer F.Cu) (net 6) (status 10))
 (segment (start 154.5 87.735) (end 154.5 87.25) (width 1) (layer F.Cu) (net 6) (status 30))
 (segment (start 150.85 91.385) (end 154.5 87.735) (width 1) (layer F.Cu) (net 6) (status 30))
 (segment (start 162.68499 109.81501) (end 163.450001 109.049999) (width 1) (layer F.Cu) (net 4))
 (segment (start 149.68499 109.81501) (end 162.68499 109.81501) (width 1) (layer F.Cu) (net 4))
 (segment (start 163.450001 109.049999) (end 164.25 108.25) (width 1) (layer F.Cu) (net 4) (status 20))
 (segment (start 147.75 111.75) (end 149.68499 109.81501) (width 1) (layer F.Cu) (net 4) (status 10))
 (segment (start 160.200001 107.450001) (end 161 108.25) (width 1) (layer F.Cu) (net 5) (status 20))
 (segment (start 157.75 105) (end 160.200001 107.450001) (width 1) (layer F.Cu) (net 5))
 (segment (start 149.586508 105) (end 157.75 105) (width 1) (layer F.Cu) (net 5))
 (segment (start 144.25 110.336508) (end 149.586508 105) (width 1) (layer F.Cu) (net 5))
 (segment (start 144.25 111.75) (end 144.25 110.336508) (width 1) (layer F.Cu) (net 5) (status 10))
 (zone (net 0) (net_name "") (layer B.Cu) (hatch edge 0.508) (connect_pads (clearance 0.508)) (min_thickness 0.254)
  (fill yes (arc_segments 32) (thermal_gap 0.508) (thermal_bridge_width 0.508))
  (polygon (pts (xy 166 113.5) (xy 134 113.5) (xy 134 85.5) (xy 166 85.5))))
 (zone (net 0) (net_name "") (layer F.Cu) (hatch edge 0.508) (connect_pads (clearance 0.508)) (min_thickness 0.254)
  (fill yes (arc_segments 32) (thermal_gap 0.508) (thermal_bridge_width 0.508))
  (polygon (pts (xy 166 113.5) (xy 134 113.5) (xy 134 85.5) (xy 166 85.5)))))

